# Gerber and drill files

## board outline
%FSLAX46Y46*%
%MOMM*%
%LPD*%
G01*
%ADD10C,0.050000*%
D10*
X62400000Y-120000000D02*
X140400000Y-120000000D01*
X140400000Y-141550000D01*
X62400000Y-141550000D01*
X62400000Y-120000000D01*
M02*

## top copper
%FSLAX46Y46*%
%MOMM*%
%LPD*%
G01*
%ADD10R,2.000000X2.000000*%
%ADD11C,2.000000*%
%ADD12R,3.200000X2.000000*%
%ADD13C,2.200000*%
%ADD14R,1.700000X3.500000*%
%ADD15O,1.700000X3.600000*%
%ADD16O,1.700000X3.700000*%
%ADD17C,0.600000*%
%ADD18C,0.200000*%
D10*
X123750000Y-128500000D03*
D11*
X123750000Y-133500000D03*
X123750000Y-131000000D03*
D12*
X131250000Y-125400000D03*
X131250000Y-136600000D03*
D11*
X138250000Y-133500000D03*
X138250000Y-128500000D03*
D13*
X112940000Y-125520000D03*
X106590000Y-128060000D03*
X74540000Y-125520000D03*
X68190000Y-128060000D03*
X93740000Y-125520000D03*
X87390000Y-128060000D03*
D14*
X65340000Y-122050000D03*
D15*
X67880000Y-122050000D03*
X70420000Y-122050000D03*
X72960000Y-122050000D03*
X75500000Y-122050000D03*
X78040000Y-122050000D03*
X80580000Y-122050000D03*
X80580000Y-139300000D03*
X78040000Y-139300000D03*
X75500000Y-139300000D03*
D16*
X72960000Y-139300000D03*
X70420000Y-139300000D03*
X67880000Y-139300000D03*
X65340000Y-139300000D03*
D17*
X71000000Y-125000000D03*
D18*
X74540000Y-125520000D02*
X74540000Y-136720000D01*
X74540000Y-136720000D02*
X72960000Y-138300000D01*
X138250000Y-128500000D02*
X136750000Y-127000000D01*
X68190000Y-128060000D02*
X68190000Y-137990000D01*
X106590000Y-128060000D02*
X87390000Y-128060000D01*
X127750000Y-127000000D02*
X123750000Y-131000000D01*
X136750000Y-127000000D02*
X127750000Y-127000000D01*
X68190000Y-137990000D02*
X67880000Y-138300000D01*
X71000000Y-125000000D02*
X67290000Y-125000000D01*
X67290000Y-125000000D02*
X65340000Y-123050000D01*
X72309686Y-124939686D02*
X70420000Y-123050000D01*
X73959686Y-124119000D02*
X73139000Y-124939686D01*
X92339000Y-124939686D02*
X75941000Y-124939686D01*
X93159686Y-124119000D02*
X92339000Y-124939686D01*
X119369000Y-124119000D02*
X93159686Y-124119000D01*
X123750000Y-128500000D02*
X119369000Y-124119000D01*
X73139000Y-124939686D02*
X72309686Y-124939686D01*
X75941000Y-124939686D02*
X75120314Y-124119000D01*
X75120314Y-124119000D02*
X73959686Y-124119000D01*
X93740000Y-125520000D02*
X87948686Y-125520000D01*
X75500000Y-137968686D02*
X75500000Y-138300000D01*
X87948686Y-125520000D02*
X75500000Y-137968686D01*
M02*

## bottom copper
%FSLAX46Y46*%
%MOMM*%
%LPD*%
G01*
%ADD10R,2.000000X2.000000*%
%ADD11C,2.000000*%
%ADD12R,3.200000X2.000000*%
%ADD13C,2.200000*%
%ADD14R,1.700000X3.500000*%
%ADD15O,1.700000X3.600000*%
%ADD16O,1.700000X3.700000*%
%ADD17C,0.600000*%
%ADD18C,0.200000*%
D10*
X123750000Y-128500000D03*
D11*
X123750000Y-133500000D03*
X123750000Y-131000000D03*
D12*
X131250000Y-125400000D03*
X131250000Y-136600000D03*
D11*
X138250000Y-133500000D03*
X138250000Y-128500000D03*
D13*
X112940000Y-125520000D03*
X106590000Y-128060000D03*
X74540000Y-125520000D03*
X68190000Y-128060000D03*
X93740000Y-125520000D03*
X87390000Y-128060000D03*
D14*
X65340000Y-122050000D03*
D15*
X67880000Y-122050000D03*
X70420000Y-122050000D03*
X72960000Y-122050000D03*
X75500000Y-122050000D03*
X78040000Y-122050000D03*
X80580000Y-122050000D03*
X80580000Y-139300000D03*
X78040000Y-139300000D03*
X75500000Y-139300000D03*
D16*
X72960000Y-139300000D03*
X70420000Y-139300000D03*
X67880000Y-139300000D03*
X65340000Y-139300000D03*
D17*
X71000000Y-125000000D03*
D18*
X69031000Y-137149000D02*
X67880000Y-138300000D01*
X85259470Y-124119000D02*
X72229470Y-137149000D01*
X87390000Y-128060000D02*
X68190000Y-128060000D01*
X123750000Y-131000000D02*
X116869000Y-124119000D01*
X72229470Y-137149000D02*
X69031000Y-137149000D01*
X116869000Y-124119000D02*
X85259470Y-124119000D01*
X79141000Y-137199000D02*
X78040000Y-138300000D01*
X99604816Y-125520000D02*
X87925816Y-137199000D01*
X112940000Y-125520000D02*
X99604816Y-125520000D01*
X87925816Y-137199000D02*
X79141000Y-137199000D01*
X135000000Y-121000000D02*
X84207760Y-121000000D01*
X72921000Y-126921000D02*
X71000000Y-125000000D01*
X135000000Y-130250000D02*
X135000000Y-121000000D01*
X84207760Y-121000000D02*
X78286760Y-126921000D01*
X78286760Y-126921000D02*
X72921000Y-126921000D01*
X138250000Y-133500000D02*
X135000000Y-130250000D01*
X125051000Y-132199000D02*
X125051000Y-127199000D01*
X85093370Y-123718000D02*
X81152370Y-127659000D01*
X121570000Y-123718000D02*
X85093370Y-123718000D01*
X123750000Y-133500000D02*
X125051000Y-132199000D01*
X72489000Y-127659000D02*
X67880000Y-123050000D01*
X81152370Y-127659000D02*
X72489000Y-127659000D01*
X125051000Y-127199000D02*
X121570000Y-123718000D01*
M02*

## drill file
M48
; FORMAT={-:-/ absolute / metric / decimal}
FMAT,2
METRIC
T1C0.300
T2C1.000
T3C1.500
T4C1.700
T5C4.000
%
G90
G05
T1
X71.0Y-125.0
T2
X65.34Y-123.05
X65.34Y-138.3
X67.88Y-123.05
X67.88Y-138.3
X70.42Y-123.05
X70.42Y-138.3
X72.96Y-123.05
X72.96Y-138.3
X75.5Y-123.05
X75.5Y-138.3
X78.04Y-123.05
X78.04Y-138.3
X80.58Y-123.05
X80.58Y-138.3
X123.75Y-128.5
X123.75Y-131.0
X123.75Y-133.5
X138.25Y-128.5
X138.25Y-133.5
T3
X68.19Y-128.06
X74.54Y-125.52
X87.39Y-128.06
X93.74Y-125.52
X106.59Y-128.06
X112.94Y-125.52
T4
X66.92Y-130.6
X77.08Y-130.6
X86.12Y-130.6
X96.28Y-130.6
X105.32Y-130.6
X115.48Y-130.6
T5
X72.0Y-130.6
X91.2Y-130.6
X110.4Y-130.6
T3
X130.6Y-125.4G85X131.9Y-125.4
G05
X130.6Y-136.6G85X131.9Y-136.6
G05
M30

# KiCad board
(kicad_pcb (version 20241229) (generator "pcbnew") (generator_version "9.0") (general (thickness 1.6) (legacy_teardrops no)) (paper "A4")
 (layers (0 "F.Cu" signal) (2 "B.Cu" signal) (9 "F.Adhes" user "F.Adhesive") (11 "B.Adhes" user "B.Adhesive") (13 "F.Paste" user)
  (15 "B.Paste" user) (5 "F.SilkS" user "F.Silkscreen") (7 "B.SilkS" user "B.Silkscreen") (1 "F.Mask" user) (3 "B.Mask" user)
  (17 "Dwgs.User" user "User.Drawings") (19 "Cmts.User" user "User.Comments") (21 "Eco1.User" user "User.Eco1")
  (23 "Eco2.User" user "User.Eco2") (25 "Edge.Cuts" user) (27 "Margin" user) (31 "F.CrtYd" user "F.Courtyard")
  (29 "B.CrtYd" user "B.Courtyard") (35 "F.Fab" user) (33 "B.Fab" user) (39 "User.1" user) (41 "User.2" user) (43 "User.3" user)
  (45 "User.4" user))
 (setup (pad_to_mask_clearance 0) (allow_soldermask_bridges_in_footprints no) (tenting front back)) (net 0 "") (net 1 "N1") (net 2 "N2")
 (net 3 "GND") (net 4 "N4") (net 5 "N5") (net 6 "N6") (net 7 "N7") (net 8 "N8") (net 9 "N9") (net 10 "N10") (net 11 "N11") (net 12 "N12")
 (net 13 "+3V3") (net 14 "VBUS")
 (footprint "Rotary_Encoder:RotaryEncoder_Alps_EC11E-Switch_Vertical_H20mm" (layer "F.Cu") (at 123.75 128.5)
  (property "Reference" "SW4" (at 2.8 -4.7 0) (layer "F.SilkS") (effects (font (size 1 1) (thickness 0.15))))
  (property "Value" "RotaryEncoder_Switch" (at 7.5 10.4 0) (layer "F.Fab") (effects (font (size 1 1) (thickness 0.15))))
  (pad "A" thru_hole rect (at 0 0) (size 2 2) (drill 1) (layers "*.Cu" "*.Mask") (remove_unused_layers no) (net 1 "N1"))
  (pad "B" thru_hole circle (at 0 5) (size 2 2) (drill 1) (layers "*.Cu" "*.Mask") (remove_unused_layers no) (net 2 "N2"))
  (pad "C" thru_hole circle (at 0 2.5) (size 2 2) (drill 1) (layers "*.Cu" "*.Mask") (remove_unused_layers no) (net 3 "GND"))
  (pad "MP" thru_hole rect (at 7.5 -3.1) (size 3.2 2) (drill oval 2.8 1.5) (layers "*.Cu" "*.Mask") (remove_unused_layers no))
  (pad "MP" thru_hole rect (at 7.5 8.1) (size 3.2 2) (drill oval 2.8 1.5) (layers "*.Cu" "*.Mask") (remove_unused_layers no))
  (pad "S1" thru_hole circle (at 14.5 5) (size 2 2) (drill 1) (layers "*.Cu" "*.Mask") (remove_unused_layers no) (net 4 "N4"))
  (pad "S2" thru_hole circle (at 14.5 0) (size 2 2) (drill 1) (layers "*.Cu" "*.Mask") (remove_unused_layers no) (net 3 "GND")))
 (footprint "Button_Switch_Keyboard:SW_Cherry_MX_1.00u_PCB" (layer "F.Cu") (at 112.94 125.52)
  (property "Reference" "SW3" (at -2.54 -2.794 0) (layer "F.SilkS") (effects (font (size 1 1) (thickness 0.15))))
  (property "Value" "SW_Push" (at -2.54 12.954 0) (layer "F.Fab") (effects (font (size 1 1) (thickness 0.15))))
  (pad "" np_thru_hole circle (at -7.62 5.08) (size 1.7 1.7) (drill 1.7) (layers "*.Cu" "*.Mask"))
  (pad "" np_thru_hole circle (at -2.54 5.08) (size 4 4) (drill 4) (layers "*.Cu" "*.Mask"))
  (pad "" np_thru_hole circle (at 2.54 5.08) (size 1.7 1.7) (drill 1.7) (layers "*.Cu" "*.Mask"))
  (pad "1" thru_hole circle (at 0 0) (size 2.2 2.2) (drill 1.5) (layers "*.Cu" "*.Mask") (remove_unused_layers no) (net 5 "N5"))
  (pad "2" thru_hole circle (at -6.35 2.54) (size 2.2 2.2) (drill 1.5) (layers "*.Cu" "*.Mask") (remove_unused_layers no) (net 3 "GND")))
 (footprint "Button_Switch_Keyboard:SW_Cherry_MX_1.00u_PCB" (layer "F.Cu") (at 74.54 125.52)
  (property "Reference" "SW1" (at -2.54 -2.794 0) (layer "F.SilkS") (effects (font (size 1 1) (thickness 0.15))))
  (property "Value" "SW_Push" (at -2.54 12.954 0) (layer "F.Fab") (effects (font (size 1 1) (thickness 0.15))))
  (pad "" np_thru_hole circle (at -7.62 5.08) (size 1.7 1.7) (drill 1.7) (layers "*.Cu" "*.Mask"))
  (pad "" np_thru_hole circle (at -2.54 5.08) (size 4 4) (drill 4) (layers "*.Cu" "*.Mask"))
  (pad "" np_thru_hole circle (at 2.54 5.08) (size 1.7 1.7) (drill 1.7) (layers "*.Cu" "*.Mask"))
  (pad "1" thru_hole circle (at 0 0) (size 2.2 2.2) (drill 1.5) (layers "*.Cu" "*.Mask") (remove_unused_layers no) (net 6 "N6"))
  (pad "2" thru_hole circle (at -6.35 2.54) (size 2.2 2.2) (drill 1.5) (layers "*.Cu" "*.Mask") (remove_unused_layers no) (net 3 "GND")))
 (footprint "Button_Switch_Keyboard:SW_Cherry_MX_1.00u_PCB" (layer "F.Cu") (at 93.74 125.52)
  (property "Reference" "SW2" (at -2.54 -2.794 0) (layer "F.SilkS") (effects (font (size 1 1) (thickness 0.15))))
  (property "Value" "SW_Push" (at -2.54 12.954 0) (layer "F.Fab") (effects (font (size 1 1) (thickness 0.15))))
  (pad "" np_thru_hole circle (at -7.62 5.08) (size 1.7 1.7) (drill 1.7) (layers "*.Cu" "*.Mask"))
  (pad "" np_thru_hole circle (at -2.54 5.08) (size 4 4) (drill 4) (layers "*.Cu" "*.Mask"))
  (pad "" np_thru_hole circle (at 2.54 5.08) (size 1.7 1.7) (drill 1.7) (layers "*.Cu" "*.Mask"))
  (pad "1" thru_hole circle (at 0 0) (size 2.2 2.2) (drill 1.5) (layers "*.Cu" "*.Mask") (remove_unused_layers no) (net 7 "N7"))
  (pad "2" thru_hole circle (at -6.35 2.54) (size 2.2 2.2) (drill 1.5) (layers "*.Cu" "*.Mask") (remove_unused_layers no) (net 3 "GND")))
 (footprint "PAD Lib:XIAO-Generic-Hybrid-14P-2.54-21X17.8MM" (layer "B.Cu") (at 72.96 130.675 -90)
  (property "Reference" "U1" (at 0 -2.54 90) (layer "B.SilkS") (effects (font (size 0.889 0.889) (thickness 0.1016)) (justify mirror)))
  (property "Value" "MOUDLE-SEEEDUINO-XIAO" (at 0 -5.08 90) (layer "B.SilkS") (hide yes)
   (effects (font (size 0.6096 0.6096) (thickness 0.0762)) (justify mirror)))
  (pad "1" thru_hole rect (at -7.625 7.62 270) (size 3.5 1.7) (drill 1 (offset -1 0)) (layers "*.Cu" "*.Mask") (remove_unused_layers no)
   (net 4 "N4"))
  (pad "2" thru_hole oval (at -7.625 5.08 270) (size 3.6 1.7) (drill 1 (offset -1 0)) (layers "*.Cu" "*.Mask") (remove_unused_layers no)
   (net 2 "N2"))
  (pad "3" thru_hole oval (at -7.625 2.54 270) (size 3.6 1.7) (drill 1 (offset -1 0)) (layers "*.Cu" "*.Mask") (remove_unused_layers no)
   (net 1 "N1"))
  (pad "4" thru_hole oval (at -7.625 0 270) (size 3.6 1.7) (drill 1 (offset -1 0)) (layers "*.Cu" "*.Mask") (remove_unused_layers no)
   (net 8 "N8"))
  (pad "5" thru_hole oval (at -7.625 -2.54 270) (size 3.6 1.7) (drill 1 (offset -1 0)) (layers "*.Cu" "*.Mask") (remove_unused_layers no)
   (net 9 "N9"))
  (pad "6" thru_hole oval (at -7.625 -5.08 90) (size 3.6 1.7) (drill 1 (offset 1 0)) (layers "*.Cu" "*.Mask") (remove_unused_layers no)
   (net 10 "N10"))
  (pad "7" thru_hole oval (at -7.625 -7.62 270) (size 3.6 1.7) (drill 1 (offset -1 0)) (layers "*.Cu" "*.Mask") (remove_unused_layers no)
   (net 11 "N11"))
  (pad "8" thru_hole oval (at 7.625 -7.62 270) (size 3.6 1.7) (drill 1 (offset 1 0)) (layers "*.Cu" "*.Mask") (remove_unused_layers no)
   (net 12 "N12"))
  (pad "9" thru_hole oval (at 7.625 -5.08 270) (size 3.6 1.7) (drill 1 (offset 1 0)) (layers "*.Cu" "*.Mask") (remove_unused_layers no)
   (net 5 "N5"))
  (pad "10" thru_hole oval (at 7.625 -2.54 270) (size 3.6 1.7) (drill 1 (offset 1 0)) (layers "*.Cu" "*.Mask") (remove_unused_layers no)
   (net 7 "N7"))
  (pad "11" thru_hole oval (at 7.625 0 270) (size 3.7 1.7) (drill 1 (offset 1 0)) (layers "*.Cu" "*.Mask") (remove_unused_layers no)
   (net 6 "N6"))
  (pad "12" thru_hole oval (at 7.625 2.54 270) (size 3.7 1.7) (drill 1 (offset 1 0)) (layers "*.Cu" "*.Mask") (remove_unused_layers no)
   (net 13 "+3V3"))
  (pad "13" thru_hole oval (at 7.625 5.08 270) (size 3.7 1.7) (drill 1 (offset 1 0)) (layers "*.Cu" "*.Mask") (remove_unused_layers no)
   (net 3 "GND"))
  (pad "14" thru_hole oval (at 7.625 7.62 270) (size 3.7 1.7) (drill 1 (offset 1 0)) (layers "*.Cu" "*.Mask") (remove_unused_layers no)
   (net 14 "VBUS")))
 (gr_rect (start 62.4 120) (end 140.4 141.55) (stroke (width 0.05) (type default)) (fill no) (layer "Edge.Cuts"))
 (segment (start 74.54 125.52) (end 74.54 136.72) (width 0.2) (layer "F.Cu") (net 6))
 (segment (start 74.54 136.72) (end 72.96 138.3) (width 0.2) (layer "F.Cu") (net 6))
 (segment (start 138.25 128.5) (end 136.75 127) (width 0.2) (layer "F.Cu") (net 3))
 (segment (start 68.19 128.06) (end 68.19 137.99) (width 0.2) (layer "F.Cu") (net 3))
 (segment (start 106.59 128.06) (end 87.39 128.06) (width 0.2) (layer "F.Cu") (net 3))
 (segment (start 127.75 127) (end 123.75 131) (width 0.2) (layer "F.Cu") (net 3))
 (segment (start 136.75 127) (end 127.75 127) (width 0.2) (layer "F.Cu") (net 3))
 (segment (start 68.19 137.99) (end 67.88 138.3) (width 0.2) (layer "F.Cu") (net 3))
 (segment (start 69.031 137.149) (end 67.88 138.3) (width 0.2) (layer "B.Cu") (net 3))
 (segment (start 85.25947 124.119) (end 72.22947 137.149) (width 0.2) (layer "B.Cu") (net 3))
 (segment (start 87.39 128.06) (end 68.19 128.06) (width 0.2) (layer "B.Cu") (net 3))
 (segment (start 123.75 131) (end 116.869 124.119) (width 0.2) (layer "B.Cu") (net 3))
 (segment (start 72.22947 137.149) (end 69.031 137.149) (width 0.2) (layer "B.Cu") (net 3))
 (segment (start 116.869 124.119) (end 85.25947 124.119) (width 0.2) (layer "B.Cu") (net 3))
 (segment (start 79.141 137.199) (end 78.04 138.3) (width 0.2) (layer "B.Cu") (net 5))
 (segment (start 99.604816 125.52) (end 87.925816 137.199) (width 0.2) (layer "B.Cu") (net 5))
 (segment (start 112.94 125.52) (end 99.604816 125.52) (width 0.2) (layer "B.Cu") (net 5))
 (segment (start 87.925816 137.199) (end 79.141 137.199) (width 0.2) (layer "B.Cu") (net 5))
 (segment (start 71 125) (end 67.29 125) (width 0.2) (layer "F.Cu") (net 4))
 (segment (start 67.29 125) (end 65.34 123.05) (width 0.2) (layer "F.Cu") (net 4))
 (via (at 71 125) (size 0.6) (drill 0.3) (layers "F.Cu" "B.Cu") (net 4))
 (segment (start 135 121) (end 84.20776 121) (width 0.2) (layer "B.Cu") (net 4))
 (segment (start 72.921 126.921) (end 71 125) (width 0.2) (layer "B.Cu") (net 4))
 (segment (start 135 130.25) (end 135 121) (width 0.2) (layer "B.Cu") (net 4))
 (segment (start 84.20776 121) (end 78.28676 126.921) (width 0.2) (layer "B.Cu") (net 4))
 (segment (start 78.28676 126.921) (end 72.921 126.921) (width 0.2) (layer "B.Cu") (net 4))
 (segment (start 138.25 133.5) (end 135 130.25) (width 0.2) (layer "B.Cu") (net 4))
 (segment (start 72.309686 124.939686) (end 70.42 123.05) (width 0.2) (layer "F.Cu") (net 1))
 (segment (start 73.959686 124.119) (end 73.139 124.939686) (width 0.2) (layer "F.Cu") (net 1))
 (segment (start 92.339 124.939686) (end 75.941 124.939686) (width 0.2) (layer "F.Cu") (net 1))
 (segment (start 93.159686 124.119) (end 92.339 124.939686) (width 0.2) (layer "F.Cu") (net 1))
 (segment (start 119.369 124.119) (end 93.159686 124.119) (width 0.2) (layer "F.Cu") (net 1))
 (segment (start 123.75 128.5) (end 119.369 124.119) (width 0.2) (layer "F.Cu") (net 1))
 (segment (start 73.139 124.939686) (end 72.309686 124.939686) (width 0.2) (layer "F.Cu") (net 1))
 (segment (start 75.941 124.939686) (end 75.120314 124.119) (width 0.2) (layer "F.Cu") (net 1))
 (segment (start 75.120314 124.119) (end 73.959686 124.119) (width 0.2) (layer "F.Cu") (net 1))
 (segment (start 93.74 125.52) (end 87.948686 125.52) (width 0.2) (layer "F.Cu") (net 7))
 (segment (start 75.5 137.968686) (end 75.5 138.3) (width 0.2) (layer "F.Cu") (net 7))
 (segment (start 87.948686 125.52) (end 75.5 137.968686) (width 0.2) (layer "F.Cu") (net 7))
 (segment (start 125.051 132.199) (end 125.051 127.199) (width 0.2) (layer "B.Cu") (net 2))
 (segment (start 85.09337 123.718) (end 81.15237 127.659) (width 0.2) (layer "B.Cu") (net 2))
 (segment (start 121.57 123.718) (end 85.09337 123.718) (width 0.2) (layer "B.Cu") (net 2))
 (segment (start 123.75 133.5) (end 125.051 132.199) (width 0.2) (layer "B.Cu") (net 2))
 (segment (start 72.489 127.659) (end 67.88 123.05) (width 0.2) (layer "B.Cu") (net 2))
 (segment (start 81.15237 127.659) (end 72.489 127.659) (width 0.2) (layer "B.Cu") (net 2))
 (segment (start 125.051 127.199) (end 121.57 123.718) (width 0.2) (layer "B.Cu") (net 2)))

